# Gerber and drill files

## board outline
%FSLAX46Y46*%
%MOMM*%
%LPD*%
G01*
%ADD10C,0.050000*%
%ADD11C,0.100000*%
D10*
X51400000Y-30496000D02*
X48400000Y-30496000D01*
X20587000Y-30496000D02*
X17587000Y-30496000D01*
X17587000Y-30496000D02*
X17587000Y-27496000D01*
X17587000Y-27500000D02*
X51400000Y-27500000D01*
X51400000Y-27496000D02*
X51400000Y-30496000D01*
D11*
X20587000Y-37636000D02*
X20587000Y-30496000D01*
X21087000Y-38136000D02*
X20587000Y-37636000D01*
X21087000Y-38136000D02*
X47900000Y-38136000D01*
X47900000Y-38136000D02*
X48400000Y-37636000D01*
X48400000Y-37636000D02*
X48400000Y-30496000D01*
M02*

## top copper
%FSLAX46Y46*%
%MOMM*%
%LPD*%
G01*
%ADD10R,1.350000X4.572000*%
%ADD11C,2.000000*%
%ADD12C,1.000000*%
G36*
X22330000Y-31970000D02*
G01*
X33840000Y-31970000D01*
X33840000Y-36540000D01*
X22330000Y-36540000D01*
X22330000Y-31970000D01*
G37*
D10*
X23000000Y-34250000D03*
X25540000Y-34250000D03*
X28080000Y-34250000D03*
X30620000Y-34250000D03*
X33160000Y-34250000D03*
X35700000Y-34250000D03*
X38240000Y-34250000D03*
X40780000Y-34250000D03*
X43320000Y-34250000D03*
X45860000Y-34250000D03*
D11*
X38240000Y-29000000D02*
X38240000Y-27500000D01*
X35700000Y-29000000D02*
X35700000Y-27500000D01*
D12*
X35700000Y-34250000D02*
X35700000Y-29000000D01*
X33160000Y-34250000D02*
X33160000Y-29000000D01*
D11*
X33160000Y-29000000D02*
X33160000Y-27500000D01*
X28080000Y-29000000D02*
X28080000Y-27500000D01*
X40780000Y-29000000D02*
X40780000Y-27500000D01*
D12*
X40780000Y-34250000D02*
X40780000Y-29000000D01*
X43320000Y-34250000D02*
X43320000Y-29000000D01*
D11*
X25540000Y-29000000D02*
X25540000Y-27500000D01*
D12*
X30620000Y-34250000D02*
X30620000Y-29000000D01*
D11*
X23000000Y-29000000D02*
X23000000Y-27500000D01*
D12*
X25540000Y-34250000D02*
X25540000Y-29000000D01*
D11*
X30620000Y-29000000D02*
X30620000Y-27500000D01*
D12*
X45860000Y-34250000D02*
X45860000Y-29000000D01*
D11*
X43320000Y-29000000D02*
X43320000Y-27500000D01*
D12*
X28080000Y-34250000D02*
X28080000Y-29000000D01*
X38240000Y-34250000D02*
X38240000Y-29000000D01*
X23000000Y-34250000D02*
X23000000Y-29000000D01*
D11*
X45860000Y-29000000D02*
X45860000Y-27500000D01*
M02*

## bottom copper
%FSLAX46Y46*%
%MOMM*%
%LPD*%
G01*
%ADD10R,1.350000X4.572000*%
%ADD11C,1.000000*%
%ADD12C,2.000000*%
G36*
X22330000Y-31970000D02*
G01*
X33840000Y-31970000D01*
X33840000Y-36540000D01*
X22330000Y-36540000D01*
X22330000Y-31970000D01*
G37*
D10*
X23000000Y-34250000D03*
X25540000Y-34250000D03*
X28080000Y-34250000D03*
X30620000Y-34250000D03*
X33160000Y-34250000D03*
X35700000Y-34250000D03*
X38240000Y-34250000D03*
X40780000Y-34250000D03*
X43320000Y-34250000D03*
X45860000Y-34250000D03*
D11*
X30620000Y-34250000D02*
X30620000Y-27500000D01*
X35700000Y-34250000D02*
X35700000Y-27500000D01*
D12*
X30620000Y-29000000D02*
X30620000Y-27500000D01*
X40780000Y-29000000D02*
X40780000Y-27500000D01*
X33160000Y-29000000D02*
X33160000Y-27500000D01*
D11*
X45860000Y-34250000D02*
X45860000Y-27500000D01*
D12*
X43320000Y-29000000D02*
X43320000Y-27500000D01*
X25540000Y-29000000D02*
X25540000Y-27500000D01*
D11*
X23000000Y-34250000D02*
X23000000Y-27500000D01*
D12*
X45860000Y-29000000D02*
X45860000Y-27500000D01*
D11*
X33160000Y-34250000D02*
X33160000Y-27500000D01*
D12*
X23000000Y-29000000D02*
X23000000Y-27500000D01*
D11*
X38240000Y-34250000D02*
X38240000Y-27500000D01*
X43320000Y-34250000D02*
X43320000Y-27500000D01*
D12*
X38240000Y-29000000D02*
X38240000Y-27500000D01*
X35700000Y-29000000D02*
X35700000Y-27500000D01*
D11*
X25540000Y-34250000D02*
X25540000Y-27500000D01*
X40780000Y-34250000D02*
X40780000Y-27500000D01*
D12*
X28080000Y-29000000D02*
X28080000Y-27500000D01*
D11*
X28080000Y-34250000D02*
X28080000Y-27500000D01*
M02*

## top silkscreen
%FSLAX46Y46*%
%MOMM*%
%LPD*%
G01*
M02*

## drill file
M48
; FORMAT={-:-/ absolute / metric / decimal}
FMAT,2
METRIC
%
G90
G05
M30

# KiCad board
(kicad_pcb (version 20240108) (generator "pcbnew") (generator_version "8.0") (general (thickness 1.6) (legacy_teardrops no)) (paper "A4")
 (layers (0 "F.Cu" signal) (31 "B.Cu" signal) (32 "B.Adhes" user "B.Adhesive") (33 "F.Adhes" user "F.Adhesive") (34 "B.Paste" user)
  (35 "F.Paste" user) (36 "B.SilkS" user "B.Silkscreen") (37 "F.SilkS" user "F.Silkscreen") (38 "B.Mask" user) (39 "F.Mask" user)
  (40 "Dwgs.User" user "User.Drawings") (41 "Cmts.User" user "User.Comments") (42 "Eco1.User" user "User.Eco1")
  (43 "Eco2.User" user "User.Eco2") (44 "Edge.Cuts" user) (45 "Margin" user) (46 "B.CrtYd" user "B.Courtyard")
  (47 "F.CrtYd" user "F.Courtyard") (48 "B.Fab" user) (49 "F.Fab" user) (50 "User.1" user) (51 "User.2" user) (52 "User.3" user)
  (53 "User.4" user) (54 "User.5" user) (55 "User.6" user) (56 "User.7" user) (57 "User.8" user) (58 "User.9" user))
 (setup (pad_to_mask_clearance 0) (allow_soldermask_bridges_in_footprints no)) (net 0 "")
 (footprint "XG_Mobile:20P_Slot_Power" (layer "F.Cu") (at 23 34.25)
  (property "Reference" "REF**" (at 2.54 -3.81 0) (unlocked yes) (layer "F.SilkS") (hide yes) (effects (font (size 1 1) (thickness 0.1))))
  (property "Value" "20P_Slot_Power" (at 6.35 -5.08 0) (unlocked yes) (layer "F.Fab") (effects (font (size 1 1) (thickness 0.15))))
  (fp_line (start -2.413 3.386) (end -2.413 -3.754) (stroke (width 0.1) (type default)) (layer "Edge.Cuts"))
  (fp_line (start -1.913 3.886) (end -2.413 3.386) (stroke (width 0.1) (type default)) (layer "Edge.Cuts"))
  (fp_line (start -1.913 3.886) (end 24.9 3.886) (stroke (width 0.1) (type default)) (layer "Edge.Cuts"))
  (fp_line (start 24.9 3.886) (end 25.4 3.386) (stroke (width 0.1) (type default)) (layer "Edge.Cuts"))
  (fp_line (start 25.4 3.386) (end 25.4 -3.754) (stroke (width 0.1) (type default)) (layer "Edge.Cuts"))
  (pad "1" smd rect (at 0 0) (size 1.35 4.572) (layers "F.Cu") (thermal_bridge_angle 45))
  (pad "2" smd rect (at 0 0) (size 1.35 4.572) (layers "B.Cu") (thermal_bridge_angle 45))
  (pad "3" smd rect (at 2.54 0) (size 1.35 4.572) (layers "F.Cu") (thermal_bridge_angle 45))
  (pad "4" smd rect (at 2.54 0) (size 1.35 4.572) (layers "B.Cu") (thermal_bridge_angle 45))
  (pad "5" smd rect (at 5.08 0) (size 1.35 4.572) (layers "F.Cu") (thermal_bridge_angle 45))
  (pad "6" smd rect (at 5.08 0) (size 1.35 4.572) (layers "B.Cu") (thermal_bridge_angle 45))
  (pad "7" smd rect (at 7.62 0) (size 1.35 4.572) (layers "F.Cu") (thermal_bridge_angle 45))
  (pad "8" smd rect (at 7.62 0) (size 1.35 4.572) (layers "B.Cu") (thermal_bridge_angle 45))
  (pad "9" smd rect (at 10.16 0) (size 1.35 4.572) (layers "F.Cu") (thermal_bridge_angle 45))
  (pad "10" smd rect (at 10.16 0) (size 1.35 4.572) (layers "B.Cu") (thermal_bridge_angle 45))
  (pad "11" smd rect (at 12.7 0) (size 1.35 4.572) (layers "F.Cu") (thermal_bridge_angle 45))
  (pad "12" smd rect (at 12.7 0) (size 1.35 4.572) (layers "B.Cu") (thermal_bridge_angle 45))
  (pad "13" smd rect (at 15.24 0) (size 1.35 4.572) (layers "F.Cu") (thermal_bridge_angle 45))
  (pad "14" smd rect (at 15.24 0) (size 1.35 4.572) (layers "B.Cu") (thermal_bridge_angle 45))
  (pad "15" smd rect (at 17.78 0) (size 1.35 4.572) (layers "F.Cu") (thermal_bridge_angle 45))
  (pad "16" smd rect (at 17.78 0) (size 1.35 4.572) (layers "B.Cu") (thermal_bridge_angle 45))
  (pad "17" smd rect (at 20.32 0) (size 1.35 4.572) (layers "F.Cu") (thermal_bridge_angle 45))
  (pad "18" smd rect (at 20.32 0) (size 1.35 4.572) (layers "B.Cu") (thermal_bridge_angle 45))
  (pad "19" smd rect (at 22.86 0) (size 1.35 4.572) (layers "F.Cu") (thermal_bridge_angle 45))
  (pad "20" smd rect (at 22.86 0) (size 1.35 4.572) (layers "B.Cu") (thermal_bridge_angle 45)))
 (gr_rect (start 22.33 31.97) (end 33.84 36.54) (stroke (width 0) (type solid)) (fill solid) (layer "F.Cu"))
 (gr_rect (start 22.33 31.97) (end 33.84 36.54) (stroke (width 0) (type solid)) (fill solid) (layer "B.Cu"))
 (gr_line (start 51.4 30.496) (end 48.4 30.496) (stroke (width 0.05) (type default)) (layer "Edge.Cuts"))
 (gr_line (start 20.587 30.496) (end 17.587 30.496) (stroke (width 0.05) (type default)) (layer "Edge.Cuts"))
 (gr_line (start 17.587 30.496) (end 17.587 27.496) (stroke (width 0.05) (type default)) (layer "Edge.Cuts"))
 (gr_line (start 17.587 27.5) (end 51.4 27.5) (stroke (width 0.05) (type default)) (layer "Edge.Cuts"))
 (gr_line (start 51.4 27.496) (end 51.4 30.496) (stroke (width 0.05) (type default)) (layer "Edge.Cuts"))
 (segment (start 38.24 29) (end 38.24 27.5) (width 2) (layer "F.Cu") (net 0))
 (segment (start 35.7 29) (end 35.7 27.5) (width 2) (layer "F.Cu") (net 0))
 (segment (start 35.7 34.25) (end 35.7 29) (width 1) (layer "F.Cu") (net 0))
 (segment (start 33.16 34.25) (end 33.16 29) (width 1) (layer "F.Cu") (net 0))
 (segment (start 33.16 29) (end 33.16 27.5) (width 2) (layer "F.Cu") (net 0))
 (segment (start 28.08 29) (end 28.08 27.5) (width 2) (layer "F.Cu") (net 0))
 (segment (start 40.78 29) (end 40.78 27.5) (width 2) (layer "F.Cu") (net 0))
 (segment (start 40.78 34.25) (end 40.78 29) (width 1) (layer "F.Cu") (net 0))
 (segment (start 43.32 34.25) (end 43.32 29) (width 1) (layer "F.Cu") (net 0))
 (segment (start 25.54 29) (end 25.54 27.5) (width 2) (layer "F.Cu") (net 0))
 (segment (start 30.62 34.25) (end 30.62 29) (width 1) (layer "F.Cu") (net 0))
 (segment (start 23 29) (end 23 27.5) (width 2) (layer "F.Cu") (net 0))
 (segment (start 25.54 34.25) (end 25.54 29) (width 1) (layer "F.Cu") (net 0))
 (segment (start 30.62 29) (end 30.62 27.5) (width 2) (layer "F.Cu") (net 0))
 (segment (start 45.86 34.25) (end 45.86 29) (width 1) (layer "F.Cu") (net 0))
 (segment (start 43.32 29) (end 43.32 27.5) (width 2) (layer "F.Cu") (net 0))
 (segment (start 28.08 34.25) (end 28.08 29) (width 1) (layer "F.Cu") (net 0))
 (segment (start 38.24 34.25) (end 38.24 29) (width 1) (layer "F.Cu") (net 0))
 (segment (start 23 34.25) (end 23 29) (width 1) (layer "F.Cu") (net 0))
 (segment (start 45.86 29) (end 45.86 27.5) (width 2) (layer "F.Cu") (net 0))
 (segment (start 30.62 34.25) (end 30.62 27.5) (width 1) (layer "B.Cu") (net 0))
 (segment (start 35.7 34.25) (end 35.7 27.5) (width 1) (layer "B.Cu") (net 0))
 (segment (start 30.62 29) (end 30.62 27.5) (width 2) (layer "B.Cu") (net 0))
 (segment (start 40.78 29) (end 40.78 27.5) (width 2) (layer "B.Cu") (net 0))
 (segment (start 33.16 29) (end 33.16 27.5) (width 2) (layer "B.Cu") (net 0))
 (segment (start 45.86 34.25) (end 45.86 27.5) (width 1) (layer "B.Cu") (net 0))
 (segment (start 43.32 29) (end 43.32 27.5) (width 2) (layer "B.Cu") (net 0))
 (segment (start 25.54 29) (end 25.54 27.5) (width 2) (layer "B.Cu") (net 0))
 (segment (start 23 34.25) (end 23 27.5) (width 1) (layer "B.Cu") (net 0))
 (segment (start 45.86 29) (end 45.86 27.5) (width 2) (layer "B.Cu") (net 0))
 (segment (start 33.16 34.25) (end 33.16 27.5) (width 1) (layer "B.Cu") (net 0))
 (segment (start 23 29) (end 23 27.5) (width 2) (layer "B.Cu") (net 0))
 (segment (start 38.24 34.25) (end 38.24 27.5) (width 1) (layer "B.Cu") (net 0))
 (segment (start 43.32 34.25) (end 43.32 27.5) (width 1) (layer "B.Cu") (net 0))
 (segment (start 38.24 29) (end 38.24 27.5) (width 2) (layer "B.Cu") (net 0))
 (segment (start 35.7 29) (end 35.7 27.5) (width 2) (layer "B.Cu") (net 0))
 (segment (start 25.54 34.25) (end 25.54 27.5) (width 1) (layer "B.Cu") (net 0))
 (segment (start 40.78 34.25) (end 40.78 27.5) (width 1) (layer "B.Cu") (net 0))
 (segment (start 28.08 29) (end 28.08 27.5) (width 2) (layer "B.Cu") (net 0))
 (segment (start 28.08 34.25) (end 28.08 27.5) (width 1) (layer "B.Cu") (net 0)))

